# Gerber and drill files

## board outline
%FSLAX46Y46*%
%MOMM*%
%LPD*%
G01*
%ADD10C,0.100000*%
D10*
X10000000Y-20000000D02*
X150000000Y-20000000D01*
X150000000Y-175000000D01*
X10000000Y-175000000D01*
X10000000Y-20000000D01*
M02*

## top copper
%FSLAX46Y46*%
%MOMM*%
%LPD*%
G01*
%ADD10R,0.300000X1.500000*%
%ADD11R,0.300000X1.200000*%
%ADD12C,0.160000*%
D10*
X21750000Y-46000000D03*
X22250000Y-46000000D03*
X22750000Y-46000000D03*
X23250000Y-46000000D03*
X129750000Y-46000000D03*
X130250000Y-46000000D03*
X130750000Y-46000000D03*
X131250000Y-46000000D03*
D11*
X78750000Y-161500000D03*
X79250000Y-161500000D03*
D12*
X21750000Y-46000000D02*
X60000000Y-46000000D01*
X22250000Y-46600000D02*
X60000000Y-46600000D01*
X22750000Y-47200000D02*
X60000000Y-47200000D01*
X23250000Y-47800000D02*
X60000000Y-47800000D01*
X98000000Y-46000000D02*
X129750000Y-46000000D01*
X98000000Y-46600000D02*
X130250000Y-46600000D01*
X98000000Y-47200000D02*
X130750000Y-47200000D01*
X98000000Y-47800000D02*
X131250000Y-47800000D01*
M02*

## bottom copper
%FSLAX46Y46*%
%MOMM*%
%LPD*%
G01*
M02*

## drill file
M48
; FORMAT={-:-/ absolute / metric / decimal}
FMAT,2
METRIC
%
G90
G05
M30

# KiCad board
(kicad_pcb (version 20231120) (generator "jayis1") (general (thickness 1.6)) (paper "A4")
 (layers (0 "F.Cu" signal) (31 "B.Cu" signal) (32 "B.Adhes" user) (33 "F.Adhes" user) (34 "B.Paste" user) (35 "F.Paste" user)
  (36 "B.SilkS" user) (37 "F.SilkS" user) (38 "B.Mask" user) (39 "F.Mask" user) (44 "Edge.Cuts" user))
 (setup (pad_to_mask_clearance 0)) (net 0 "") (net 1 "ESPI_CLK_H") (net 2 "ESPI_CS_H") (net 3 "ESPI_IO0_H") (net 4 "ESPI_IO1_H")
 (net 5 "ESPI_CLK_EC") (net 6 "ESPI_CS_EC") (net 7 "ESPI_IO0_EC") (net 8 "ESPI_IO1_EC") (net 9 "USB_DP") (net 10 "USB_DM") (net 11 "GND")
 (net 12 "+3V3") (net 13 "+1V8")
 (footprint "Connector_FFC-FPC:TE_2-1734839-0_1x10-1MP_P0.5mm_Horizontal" (layer "F.Cu") (at 24 46)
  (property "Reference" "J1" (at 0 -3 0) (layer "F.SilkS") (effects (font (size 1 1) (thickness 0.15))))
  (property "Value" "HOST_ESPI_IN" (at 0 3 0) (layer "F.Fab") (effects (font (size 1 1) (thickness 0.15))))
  (pad "1" smd rect (at -2.25 0) (size 0.3 1.5) (layers "F.Cu" "F.Paste" "F.Mask") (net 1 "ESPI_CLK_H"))
  (pad "2" smd rect (at -1.75 0) (size 0.3 1.5) (layers "F.Cu" "F.Paste" "F.Mask") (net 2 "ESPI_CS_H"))
  (pad "3" smd rect (at -1.25 0) (size 0.3 1.5) (layers "F.Cu" "F.Paste" "F.Mask") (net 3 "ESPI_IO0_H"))
  (pad "4" smd rect (at -0.75 0) (size 0.3 1.5) (layers "F.Cu" "F.Paste" "F.Mask") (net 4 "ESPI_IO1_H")))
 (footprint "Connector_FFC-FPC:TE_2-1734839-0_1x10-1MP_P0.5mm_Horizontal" (layer "F.Cu") (at 132 46)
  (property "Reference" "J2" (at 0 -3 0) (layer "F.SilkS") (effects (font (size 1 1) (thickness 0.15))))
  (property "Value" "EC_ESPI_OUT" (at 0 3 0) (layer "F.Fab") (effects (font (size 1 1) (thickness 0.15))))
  (pad "1" smd rect (at -2.25 0) (size 0.3 1.5) (layers "F.Cu" "F.Paste" "F.Mask") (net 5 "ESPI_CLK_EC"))
  (pad "2" smd rect (at -1.75 0) (size 0.3 1.5) (layers "F.Cu" "F.Paste" "F.Mask") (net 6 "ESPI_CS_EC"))
  (pad "3" smd rect (at -1.25 0) (size 0.3 1.5) (layers "F.Cu" "F.Paste" "F.Mask") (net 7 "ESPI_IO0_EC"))
  (pad "4" smd rect (at -0.75 0) (size 0.3 1.5) (layers "F.Cu" "F.Paste" "F.Mask") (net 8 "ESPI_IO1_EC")))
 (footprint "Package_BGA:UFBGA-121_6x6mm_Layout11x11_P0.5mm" (layer "F.Cu") (at 79 72)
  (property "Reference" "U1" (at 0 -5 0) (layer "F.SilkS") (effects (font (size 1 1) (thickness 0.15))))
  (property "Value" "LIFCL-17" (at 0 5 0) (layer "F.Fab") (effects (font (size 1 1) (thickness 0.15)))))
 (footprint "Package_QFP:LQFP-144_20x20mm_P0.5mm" (layer "F.Cu") (at 81 120)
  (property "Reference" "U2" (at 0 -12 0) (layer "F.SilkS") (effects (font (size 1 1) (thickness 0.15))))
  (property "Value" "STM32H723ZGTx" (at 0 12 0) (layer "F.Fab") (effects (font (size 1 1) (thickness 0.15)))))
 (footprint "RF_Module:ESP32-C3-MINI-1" (layer "F.Cu") (at 132 116)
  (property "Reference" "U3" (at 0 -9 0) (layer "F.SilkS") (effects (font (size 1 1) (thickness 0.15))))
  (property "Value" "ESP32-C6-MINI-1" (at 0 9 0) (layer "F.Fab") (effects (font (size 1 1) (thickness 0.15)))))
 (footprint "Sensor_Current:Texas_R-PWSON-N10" (layer "F.Cu") (at 24 118)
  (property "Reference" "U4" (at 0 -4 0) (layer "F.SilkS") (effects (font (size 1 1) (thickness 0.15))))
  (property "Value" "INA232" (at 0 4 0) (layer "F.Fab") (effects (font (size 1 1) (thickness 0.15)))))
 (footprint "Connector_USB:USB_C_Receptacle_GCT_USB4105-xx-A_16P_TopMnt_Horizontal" (layer "F.Cu") (at 80 162)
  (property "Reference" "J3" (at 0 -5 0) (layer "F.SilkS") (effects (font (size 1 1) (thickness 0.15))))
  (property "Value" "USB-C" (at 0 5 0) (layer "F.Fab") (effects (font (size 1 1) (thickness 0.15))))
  (pad "A6" smd rect (at -1.25 -0.5) (size 0.3 1.2) (layers "F.Cu" "F.Paste" "F.Mask") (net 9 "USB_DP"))
  (pad "A7" smd rect (at -0.75 -0.5) (size 0.3 1.2) (layers "F.Cu" "F.Paste" "F.Mask") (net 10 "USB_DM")))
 (segment (start 21.75 46) (end 60 46) (width 0.16) (layer "F.Cu") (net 1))
 (segment (start 22.25 46.6) (end 60 46.6) (width 0.16) (layer "F.Cu") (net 2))
 (segment (start 22.75 47.2) (end 60 47.2) (width 0.16) (layer "F.Cu") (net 3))
 (segment (start 23.25 47.8) (end 60 47.8) (width 0.16) (layer "F.Cu") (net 4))
 (segment (start 98 46) (end 129.75 46) (width 0.16) (layer "F.Cu") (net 5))
 (segment (start 98 46.6) (end 130.25 46.6) (width 0.16) (layer "F.Cu") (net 6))
 (segment (start 98 47.2) (end 130.75 47.2) (width 0.16) (layer "F.Cu") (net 7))
 (segment (start 98 47.8) (end 131.25 47.8) (width 0.16) (layer "F.Cu") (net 8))
 (gr_rect (start 10 20) (end 150 175) (stroke (width 0.1) (type default)) (fill none) (layer "Edge.Cuts")))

